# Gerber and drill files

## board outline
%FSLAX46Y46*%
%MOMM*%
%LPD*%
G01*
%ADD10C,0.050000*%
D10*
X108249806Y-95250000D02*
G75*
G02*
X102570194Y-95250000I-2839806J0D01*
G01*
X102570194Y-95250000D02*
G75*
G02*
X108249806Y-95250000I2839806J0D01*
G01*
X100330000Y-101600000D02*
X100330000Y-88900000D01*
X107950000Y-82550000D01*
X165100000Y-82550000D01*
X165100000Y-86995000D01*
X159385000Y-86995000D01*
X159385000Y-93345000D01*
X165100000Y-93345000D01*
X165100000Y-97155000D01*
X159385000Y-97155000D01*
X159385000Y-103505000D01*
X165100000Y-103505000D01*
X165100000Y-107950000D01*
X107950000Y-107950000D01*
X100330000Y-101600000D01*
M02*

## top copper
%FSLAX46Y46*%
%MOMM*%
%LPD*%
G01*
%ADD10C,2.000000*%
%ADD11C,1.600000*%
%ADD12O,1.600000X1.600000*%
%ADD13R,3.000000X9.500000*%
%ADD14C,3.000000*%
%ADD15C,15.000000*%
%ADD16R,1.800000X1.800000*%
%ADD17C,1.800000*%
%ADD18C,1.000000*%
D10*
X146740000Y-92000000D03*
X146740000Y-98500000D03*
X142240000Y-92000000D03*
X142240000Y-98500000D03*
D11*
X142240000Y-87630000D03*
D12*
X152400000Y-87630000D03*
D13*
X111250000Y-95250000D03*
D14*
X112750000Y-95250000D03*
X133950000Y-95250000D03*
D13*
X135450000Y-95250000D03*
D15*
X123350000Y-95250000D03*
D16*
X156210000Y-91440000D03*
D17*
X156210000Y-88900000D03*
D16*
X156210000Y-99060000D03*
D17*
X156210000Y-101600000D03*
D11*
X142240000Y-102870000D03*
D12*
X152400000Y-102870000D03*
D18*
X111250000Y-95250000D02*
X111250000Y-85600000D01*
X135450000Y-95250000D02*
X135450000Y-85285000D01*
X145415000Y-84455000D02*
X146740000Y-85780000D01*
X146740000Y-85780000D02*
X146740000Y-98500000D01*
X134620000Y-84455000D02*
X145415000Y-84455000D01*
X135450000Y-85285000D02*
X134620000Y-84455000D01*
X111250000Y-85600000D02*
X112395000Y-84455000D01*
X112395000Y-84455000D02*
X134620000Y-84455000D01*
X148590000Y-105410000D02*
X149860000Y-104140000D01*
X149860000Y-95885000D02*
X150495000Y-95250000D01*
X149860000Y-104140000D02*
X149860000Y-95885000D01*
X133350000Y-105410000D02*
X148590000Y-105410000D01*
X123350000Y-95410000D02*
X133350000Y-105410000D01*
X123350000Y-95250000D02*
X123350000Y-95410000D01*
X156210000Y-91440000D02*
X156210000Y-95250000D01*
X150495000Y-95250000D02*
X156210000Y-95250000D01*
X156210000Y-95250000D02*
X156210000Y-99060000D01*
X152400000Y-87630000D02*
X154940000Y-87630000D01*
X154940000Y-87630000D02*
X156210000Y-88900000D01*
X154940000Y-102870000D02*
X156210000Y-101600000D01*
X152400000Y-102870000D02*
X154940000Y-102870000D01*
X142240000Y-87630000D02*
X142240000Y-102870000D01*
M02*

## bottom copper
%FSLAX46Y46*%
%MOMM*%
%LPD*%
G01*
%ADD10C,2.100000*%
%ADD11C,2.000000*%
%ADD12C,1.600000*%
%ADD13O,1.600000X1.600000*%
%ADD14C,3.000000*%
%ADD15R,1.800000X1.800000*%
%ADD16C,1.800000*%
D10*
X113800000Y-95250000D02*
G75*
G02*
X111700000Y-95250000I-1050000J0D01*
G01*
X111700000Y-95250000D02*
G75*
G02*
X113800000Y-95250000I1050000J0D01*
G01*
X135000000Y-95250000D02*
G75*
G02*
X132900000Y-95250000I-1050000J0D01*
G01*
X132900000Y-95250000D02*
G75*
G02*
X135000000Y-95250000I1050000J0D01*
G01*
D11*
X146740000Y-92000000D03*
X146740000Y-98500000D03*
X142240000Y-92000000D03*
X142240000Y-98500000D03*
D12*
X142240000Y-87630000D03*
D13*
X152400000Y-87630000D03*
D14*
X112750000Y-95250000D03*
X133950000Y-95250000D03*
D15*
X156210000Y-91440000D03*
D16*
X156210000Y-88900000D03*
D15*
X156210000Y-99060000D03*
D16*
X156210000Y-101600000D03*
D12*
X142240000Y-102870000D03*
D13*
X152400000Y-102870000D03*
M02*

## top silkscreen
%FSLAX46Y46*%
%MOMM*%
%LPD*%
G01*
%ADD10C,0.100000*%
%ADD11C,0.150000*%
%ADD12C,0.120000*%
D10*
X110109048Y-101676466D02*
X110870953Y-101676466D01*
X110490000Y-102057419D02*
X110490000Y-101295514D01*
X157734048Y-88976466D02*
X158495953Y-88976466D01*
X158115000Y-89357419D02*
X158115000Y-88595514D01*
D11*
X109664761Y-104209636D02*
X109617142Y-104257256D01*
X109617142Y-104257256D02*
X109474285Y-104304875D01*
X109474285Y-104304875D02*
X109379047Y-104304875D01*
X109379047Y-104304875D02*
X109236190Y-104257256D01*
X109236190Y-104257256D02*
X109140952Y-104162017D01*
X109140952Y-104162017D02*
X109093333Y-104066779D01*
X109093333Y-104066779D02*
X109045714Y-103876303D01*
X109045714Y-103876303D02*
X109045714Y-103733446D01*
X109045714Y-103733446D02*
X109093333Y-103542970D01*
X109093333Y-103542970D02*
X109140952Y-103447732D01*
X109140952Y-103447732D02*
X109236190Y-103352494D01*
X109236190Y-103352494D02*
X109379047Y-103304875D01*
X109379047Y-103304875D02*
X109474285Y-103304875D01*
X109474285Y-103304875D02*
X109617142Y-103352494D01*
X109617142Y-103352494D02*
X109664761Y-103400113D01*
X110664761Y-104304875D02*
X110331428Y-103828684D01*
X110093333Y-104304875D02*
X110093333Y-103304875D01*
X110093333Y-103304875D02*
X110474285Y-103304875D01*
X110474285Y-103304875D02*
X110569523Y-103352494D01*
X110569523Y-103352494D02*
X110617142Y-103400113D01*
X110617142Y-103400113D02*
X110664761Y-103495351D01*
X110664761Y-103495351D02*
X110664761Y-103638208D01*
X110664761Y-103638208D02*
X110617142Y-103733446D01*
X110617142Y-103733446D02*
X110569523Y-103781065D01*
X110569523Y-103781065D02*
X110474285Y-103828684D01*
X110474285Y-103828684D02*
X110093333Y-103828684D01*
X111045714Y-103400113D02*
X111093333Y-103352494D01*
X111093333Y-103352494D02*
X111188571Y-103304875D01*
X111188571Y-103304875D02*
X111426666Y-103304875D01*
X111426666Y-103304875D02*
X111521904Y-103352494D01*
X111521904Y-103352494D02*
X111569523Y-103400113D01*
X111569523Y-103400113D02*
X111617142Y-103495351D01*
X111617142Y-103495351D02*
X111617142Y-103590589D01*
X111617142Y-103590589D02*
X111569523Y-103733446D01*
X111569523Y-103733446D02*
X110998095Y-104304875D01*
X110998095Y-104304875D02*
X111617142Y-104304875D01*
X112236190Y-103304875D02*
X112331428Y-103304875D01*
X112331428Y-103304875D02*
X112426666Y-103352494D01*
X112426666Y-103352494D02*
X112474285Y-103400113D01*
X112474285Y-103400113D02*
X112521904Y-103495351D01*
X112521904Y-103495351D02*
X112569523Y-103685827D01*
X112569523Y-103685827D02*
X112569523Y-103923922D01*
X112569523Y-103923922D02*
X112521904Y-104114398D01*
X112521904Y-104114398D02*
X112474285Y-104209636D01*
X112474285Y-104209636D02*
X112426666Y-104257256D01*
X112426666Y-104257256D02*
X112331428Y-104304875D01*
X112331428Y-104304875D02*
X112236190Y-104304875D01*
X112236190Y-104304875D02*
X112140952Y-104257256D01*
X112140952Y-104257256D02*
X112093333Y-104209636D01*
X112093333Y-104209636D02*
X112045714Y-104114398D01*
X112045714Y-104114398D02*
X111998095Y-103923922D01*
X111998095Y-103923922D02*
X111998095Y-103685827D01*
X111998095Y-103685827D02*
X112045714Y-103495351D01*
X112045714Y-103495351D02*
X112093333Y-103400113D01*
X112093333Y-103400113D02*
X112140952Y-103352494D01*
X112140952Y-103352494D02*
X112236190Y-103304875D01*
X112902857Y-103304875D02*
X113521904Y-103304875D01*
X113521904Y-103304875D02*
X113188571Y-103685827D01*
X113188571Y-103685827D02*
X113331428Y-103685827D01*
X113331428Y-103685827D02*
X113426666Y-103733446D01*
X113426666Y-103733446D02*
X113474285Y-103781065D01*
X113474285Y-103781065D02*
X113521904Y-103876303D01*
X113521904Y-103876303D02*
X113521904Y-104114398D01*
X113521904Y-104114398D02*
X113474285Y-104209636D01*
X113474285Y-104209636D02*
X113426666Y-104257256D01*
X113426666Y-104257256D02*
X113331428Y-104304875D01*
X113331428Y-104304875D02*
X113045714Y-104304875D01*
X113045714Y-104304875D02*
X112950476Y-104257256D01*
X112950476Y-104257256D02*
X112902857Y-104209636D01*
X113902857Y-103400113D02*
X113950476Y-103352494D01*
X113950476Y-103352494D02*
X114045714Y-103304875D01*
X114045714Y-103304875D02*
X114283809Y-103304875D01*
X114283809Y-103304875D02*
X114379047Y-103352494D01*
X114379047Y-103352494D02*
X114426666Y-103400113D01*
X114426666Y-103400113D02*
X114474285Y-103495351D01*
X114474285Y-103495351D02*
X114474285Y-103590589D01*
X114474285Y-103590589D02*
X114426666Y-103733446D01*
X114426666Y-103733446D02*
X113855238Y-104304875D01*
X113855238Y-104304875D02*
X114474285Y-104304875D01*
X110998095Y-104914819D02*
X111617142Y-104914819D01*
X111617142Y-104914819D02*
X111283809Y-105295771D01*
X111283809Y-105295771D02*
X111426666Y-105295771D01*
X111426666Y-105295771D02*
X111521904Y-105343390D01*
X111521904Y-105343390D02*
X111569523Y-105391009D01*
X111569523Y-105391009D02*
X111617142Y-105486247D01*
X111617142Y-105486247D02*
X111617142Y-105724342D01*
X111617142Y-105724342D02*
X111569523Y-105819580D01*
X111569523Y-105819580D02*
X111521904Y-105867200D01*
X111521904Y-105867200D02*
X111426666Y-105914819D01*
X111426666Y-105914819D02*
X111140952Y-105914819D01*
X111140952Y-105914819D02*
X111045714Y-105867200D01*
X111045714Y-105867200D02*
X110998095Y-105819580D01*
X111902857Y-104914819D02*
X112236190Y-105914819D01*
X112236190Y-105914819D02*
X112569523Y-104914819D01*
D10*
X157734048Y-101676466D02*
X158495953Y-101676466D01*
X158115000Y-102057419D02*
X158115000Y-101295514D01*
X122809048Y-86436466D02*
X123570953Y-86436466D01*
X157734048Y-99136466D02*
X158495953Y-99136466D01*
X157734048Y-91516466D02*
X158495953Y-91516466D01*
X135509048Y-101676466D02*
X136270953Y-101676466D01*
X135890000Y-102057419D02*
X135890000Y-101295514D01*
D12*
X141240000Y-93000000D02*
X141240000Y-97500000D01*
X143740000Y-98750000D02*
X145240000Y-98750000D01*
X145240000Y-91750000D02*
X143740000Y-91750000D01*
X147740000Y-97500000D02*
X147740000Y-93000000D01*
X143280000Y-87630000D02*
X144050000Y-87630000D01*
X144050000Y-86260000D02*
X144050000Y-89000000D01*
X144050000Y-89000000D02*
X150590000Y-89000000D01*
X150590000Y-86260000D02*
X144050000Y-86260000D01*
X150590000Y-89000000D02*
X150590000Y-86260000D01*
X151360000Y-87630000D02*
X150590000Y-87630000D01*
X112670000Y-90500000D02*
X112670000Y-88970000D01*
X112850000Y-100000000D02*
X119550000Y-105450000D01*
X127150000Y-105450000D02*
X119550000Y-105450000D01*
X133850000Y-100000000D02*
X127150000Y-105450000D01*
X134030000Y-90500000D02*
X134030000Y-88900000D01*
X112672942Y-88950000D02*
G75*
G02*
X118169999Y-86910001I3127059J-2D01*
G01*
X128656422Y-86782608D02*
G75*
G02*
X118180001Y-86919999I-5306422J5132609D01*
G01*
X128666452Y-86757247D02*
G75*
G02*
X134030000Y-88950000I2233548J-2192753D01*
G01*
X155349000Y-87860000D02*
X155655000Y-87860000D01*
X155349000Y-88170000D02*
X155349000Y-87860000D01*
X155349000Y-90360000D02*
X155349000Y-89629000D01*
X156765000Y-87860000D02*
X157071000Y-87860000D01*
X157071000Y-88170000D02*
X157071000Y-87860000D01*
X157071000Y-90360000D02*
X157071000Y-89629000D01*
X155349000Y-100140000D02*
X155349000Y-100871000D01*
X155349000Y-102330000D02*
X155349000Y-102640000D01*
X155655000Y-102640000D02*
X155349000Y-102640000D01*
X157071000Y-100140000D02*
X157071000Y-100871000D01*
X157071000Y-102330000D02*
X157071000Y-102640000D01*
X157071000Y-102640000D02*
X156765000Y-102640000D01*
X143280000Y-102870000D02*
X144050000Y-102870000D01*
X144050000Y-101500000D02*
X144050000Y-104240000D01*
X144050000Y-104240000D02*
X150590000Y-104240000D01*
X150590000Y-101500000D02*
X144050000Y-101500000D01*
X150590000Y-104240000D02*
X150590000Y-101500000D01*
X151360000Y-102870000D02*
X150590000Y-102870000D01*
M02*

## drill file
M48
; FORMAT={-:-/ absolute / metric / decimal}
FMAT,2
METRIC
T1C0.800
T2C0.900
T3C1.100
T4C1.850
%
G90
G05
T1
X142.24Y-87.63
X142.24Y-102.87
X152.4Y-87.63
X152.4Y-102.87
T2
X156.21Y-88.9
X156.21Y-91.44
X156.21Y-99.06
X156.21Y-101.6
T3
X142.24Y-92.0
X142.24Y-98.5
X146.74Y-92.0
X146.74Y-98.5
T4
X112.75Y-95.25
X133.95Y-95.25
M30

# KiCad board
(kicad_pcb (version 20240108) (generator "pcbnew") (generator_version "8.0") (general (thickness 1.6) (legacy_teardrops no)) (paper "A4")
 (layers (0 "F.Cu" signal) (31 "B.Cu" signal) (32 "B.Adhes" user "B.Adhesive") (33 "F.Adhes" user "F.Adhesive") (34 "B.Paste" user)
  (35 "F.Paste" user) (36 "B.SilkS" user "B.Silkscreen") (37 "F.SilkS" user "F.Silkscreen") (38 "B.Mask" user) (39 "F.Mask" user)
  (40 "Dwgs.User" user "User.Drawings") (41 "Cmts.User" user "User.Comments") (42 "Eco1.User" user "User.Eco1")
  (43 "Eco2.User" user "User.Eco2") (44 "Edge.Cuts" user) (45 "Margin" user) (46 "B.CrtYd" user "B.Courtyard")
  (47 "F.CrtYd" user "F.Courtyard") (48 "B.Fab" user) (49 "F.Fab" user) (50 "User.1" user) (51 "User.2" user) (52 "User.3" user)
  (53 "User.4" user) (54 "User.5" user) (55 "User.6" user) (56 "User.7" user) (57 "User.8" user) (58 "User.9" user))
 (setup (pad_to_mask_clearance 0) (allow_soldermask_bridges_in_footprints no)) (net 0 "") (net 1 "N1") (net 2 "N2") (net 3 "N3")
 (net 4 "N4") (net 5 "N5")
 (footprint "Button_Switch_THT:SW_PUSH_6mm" (layer "F.Cu") (at 146.74 92 -90)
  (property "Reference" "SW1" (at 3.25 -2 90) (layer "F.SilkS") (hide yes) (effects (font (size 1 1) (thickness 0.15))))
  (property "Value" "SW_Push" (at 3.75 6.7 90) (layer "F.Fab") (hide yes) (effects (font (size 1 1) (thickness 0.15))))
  (fp_line (start 1 5.5) (end 5.5 5.5) (stroke (width 0.12) (type solid)) (layer "F.SilkS"))
  (fp_line (start 6.75 3) (end 6.75 1.5) (stroke (width 0.12) (type solid)) (layer "F.SilkS"))
  (fp_line (start -0.25 1.5) (end -0.25 3) (stroke (width 0.12) (type solid)) (layer "F.SilkS"))
  (fp_line (start 5.5 -1) (end 1 -1) (stroke (width 0.12) (type solid)) (layer "F.SilkS"))
  (pad "1" thru_hole circle (at 0 0) (size 2 2) (drill 1.1) (layers "*.Cu" "*.Mask") (remove_unused_layers no) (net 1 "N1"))
  (pad "1" thru_hole circle (at 6.5 0) (size 2 2) (drill 1.1) (layers "*.Cu" "*.Mask") (remove_unused_layers no) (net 1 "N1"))
  (pad "2" thru_hole circle (at 0 4.5) (size 2 2) (drill 1.1) (layers "*.Cu" "*.Mask") (remove_unused_layers no) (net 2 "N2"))
  (pad "2" thru_hole circle (at 6.5 4.5) (size 2 2) (drill 1.1) (layers "*.Cu" "*.Mask") (remove_unused_layers no) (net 2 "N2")))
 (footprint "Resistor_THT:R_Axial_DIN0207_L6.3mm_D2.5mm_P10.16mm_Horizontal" (layer "F.Cu") (at 142.24 87.63)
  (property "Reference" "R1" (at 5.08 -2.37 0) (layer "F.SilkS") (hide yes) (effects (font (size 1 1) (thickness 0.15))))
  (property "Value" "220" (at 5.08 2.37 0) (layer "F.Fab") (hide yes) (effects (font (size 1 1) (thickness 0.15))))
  (fp_line (start 1.04 0) (end 1.81 0) (stroke (width 0.12) (type solid)) (layer "F.SilkS"))
  (fp_line (start 1.81 -1.37) (end 1.81 1.37) (stroke (width 0.12) (type solid)) (layer "F.SilkS"))
  (fp_line (start 1.81 1.37) (end 8.35 1.37) (stroke (width 0.12) (type solid)) (layer "F.SilkS"))
  (fp_line (start 8.35 -1.37) (end 1.81 -1.37) (stroke (width 0.12) (type solid)) (layer "F.SilkS"))
  (fp_line (start 8.35 1.37) (end 8.35 -1.37) (stroke (width 0.12) (type solid)) (layer "F.SilkS"))
  (fp_line (start 9.12 0) (end 8.35 0) (stroke (width 0.12) (type solid)) (layer "F.SilkS"))
  (pad "1" thru_hole circle (at 0 0) (size 1.6 1.6) (drill 0.8) (layers "*.Cu" "*.Mask") (remove_unused_layers no) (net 2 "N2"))
  (pad "2" thru_hole oval (at 10.16 0) (size 1.6 1.6) (drill 0.8) (layers "*.Cu" "*.Mask") (remove_unused_layers no) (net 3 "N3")))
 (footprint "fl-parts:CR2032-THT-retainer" (layer "F.Cu") (at 123.35 95.25)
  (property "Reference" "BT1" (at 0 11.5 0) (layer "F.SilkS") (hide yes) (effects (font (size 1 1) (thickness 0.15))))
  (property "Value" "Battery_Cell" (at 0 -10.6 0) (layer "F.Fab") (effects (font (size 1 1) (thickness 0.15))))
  (fp_circle (center -10.6 0) (end -8.6 0) (stroke (width 0.2) (type solid)) (fill solid) (layer "B.Cu"))
  (fp_circle (center 10.6 0) (end 12.6 0) (stroke (width 0.2) (type solid)) (fill solid) (layer "B.Cu"))
  (fp_line (start -10.68 -4.75) (end -10.68 -6.28) (stroke (width 0.12) (type solid)) (layer "F.SilkS"))
  (fp_line (start -10.5 4.75) (end -3.8 10.2) (stroke (width 0.12) (type solid)) (layer "F.SilkS"))
  (fp_line (start 3.8 10.2) (end -3.8 10.2) (stroke (width 0.12) (type solid)) (layer "F.SilkS"))
  (fp_line (start 10.5 4.75) (end 3.8 10.2) (stroke (width 0.12) (type solid)) (layer "F.SilkS"))
  (fp_line (start 10.68 -4.75) (end 10.68 -6.35) (stroke (width 0.12) (type solid)) (layer "F.SilkS"))
  (fp_arc (start -10.677058 -6.3) (mid -8.637972 -9.231689) (end -5.180001 -8.339999) (stroke (width 0.12) (type solid)) (layer "F.SilkS"))
  (fp_arc (start 5.306422 -8.467392) (mid 0.096808 -6.218103) (end -5.169999 -8.330001) (stroke (width 0.12) (type solid)) (layer "F.SilkS"))
  (fp_arc (start 5.316452 -8.492753) (mid 8.734461 -9.197232) (end 10.68 -6.3) (stroke (width 0.12) (type solid)) (layer "F.SilkS"))
  (pad "1" smd rect (at -12.1 0) (size 3 9.5) (layers "F.Cu" "F.Paste" "F.Mask") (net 1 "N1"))
  (pad "1" thru_hole circle (at -10.6 0) (size 3 3) (drill 1.85) (layers "*.Cu" "*.Mask") (remove_unused_layers no) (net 1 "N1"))
  (pad "1" thru_hole circle (at 10.6 0) (size 3 3) (drill 1.85) (layers "*.Cu" "*.Mask") (remove_unused_layers no) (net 1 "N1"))
  (pad "1" smd rect (at 12.1 0) (size 3 9.5) (layers "F.Cu" "F.Paste" "F.Mask") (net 1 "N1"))
  (pad "2" smd circle (at 0 0) (size 15 15) (layers "F.Cu" "F.Paste" "F.Mask") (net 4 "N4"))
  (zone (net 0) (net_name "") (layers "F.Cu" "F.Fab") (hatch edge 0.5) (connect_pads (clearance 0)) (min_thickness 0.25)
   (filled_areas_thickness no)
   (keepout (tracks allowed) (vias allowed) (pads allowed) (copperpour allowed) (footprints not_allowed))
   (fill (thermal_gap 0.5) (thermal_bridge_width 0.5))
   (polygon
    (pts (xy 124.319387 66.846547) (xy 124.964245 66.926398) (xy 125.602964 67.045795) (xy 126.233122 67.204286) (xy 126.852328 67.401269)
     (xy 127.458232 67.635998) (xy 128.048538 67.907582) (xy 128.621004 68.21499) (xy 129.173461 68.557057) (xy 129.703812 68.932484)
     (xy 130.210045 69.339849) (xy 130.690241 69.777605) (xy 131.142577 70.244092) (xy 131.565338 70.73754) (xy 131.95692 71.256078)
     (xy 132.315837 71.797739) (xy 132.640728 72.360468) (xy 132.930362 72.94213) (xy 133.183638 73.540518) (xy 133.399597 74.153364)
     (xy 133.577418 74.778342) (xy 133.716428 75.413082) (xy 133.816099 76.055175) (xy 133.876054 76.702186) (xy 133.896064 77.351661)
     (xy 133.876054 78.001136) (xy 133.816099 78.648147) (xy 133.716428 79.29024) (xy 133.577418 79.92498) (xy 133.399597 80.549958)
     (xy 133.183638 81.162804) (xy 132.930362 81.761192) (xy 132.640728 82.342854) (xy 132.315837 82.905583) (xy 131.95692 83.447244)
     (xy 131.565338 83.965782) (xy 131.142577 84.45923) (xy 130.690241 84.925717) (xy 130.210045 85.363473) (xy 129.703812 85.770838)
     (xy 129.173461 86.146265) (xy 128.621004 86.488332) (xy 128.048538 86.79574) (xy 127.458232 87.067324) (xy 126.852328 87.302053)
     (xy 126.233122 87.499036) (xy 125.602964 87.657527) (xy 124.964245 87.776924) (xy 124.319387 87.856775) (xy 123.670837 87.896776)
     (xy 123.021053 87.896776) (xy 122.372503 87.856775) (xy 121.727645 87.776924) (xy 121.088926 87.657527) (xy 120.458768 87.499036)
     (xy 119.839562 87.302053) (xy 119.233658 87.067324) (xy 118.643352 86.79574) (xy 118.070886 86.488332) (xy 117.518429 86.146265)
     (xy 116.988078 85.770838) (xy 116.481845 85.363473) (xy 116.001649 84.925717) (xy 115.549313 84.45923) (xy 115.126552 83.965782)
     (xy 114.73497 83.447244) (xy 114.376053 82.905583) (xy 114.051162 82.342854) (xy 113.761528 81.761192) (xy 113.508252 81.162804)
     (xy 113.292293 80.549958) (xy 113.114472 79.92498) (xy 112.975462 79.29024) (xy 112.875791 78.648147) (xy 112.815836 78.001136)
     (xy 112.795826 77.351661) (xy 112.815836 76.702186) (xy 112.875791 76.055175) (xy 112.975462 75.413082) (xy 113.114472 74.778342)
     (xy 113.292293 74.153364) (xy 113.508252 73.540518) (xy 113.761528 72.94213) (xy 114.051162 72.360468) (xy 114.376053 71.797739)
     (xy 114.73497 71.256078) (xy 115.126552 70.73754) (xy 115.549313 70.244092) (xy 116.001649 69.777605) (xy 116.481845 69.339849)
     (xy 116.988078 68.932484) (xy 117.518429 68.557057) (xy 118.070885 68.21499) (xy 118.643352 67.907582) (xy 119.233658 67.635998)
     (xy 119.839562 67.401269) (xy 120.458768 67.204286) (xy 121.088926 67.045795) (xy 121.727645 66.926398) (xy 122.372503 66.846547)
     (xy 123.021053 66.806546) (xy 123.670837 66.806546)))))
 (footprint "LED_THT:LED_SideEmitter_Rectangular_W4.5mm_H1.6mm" (layer "F.Cu") (at 156.21 91.44 90)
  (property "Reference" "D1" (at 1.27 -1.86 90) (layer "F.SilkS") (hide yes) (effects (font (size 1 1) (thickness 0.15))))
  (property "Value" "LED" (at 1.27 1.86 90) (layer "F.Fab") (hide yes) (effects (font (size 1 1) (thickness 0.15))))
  (fp_line (start 3.58 -0.861) (end 3.58 -0.555) (stroke (width 0.12) (type solid)) (layer "F.SilkS"))
  (fp_line (start 3.27 -0.861) (end 3.58 -0.861) (stroke (width 0.12) (type solid)) (layer "F.SilkS"))
  (fp_line (start 1.08 -0.861) (end 1.811 -0.861) (stroke (width 0.12) (type solid)) (layer "F.SilkS"))
  (fp_line (start 3.58 0.555) (end 3.58 0.861) (stroke (width 0.12) (type solid)) (layer "F.SilkS"))
  (fp_line (start 3.27 0.861) (end 3.58 0.861) (stroke (width 0.12) (type solid)) (layer "F.SilkS"))
  (fp_line (start 1.08 0.861) (end 1.811 0.861) (stroke (width 0.12) (type solid)) (layer "F.SilkS"))
  (pad "1" thru_hole rect (at 0 0 90) (size 1.8 1.8) (drill 0.9) (layers "*.Cu" "*.Mask") (remove_unused_layers no) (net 4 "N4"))
  (pad "2" thru_hole circle (at 2.54 0 90) (size 1.8 1.8) (drill 0.9) (layers "*.Cu" "*.Mask") (remove_unused_layers no) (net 3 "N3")))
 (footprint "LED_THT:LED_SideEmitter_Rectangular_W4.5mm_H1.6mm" (layer "F.Cu") (at 156.21 99.06 -90)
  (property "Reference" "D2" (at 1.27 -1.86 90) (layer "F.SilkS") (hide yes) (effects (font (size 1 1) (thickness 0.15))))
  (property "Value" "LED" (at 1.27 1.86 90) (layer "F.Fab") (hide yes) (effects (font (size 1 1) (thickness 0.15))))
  (fp_line (start 1.08 0.861) (end 1.811 0.861) (stroke (width 0.12) (type solid)) (layer "F.SilkS"))
  (fp_line (start 3.27 0.861) (end 3.58 0.861) (stroke (width 0.12) (type solid)) (layer "F.SilkS"))
  (fp_line (start 3.58 0.555) (end 3.58 0.861) (stroke (width 0.12) (type solid)) (layer "F.SilkS"))
  (fp_line (start 1.08 -0.861) (end 1.811 -0.861) (stroke (width 0.12) (type solid)) (layer "F.SilkS"))
  (fp_line (start 3.27 -0.861) (end 3.58 -0.861) (stroke (width 0.12) (type solid)) (layer "F.SilkS"))
  (fp_line (start 3.58 -0.861) (end 3.58 -0.555) (stroke (width 0.12) (type solid)) (layer "F.SilkS"))
  (pad "1" thru_hole rect (at 0 0 270) (size 1.8 1.8) (drill 0.9) (layers "*.Cu" "*.Mask") (remove_unused_layers no) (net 4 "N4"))
  (pad "2" thru_hole circle (at 2.54 0 270) (size 1.8 1.8) (drill 0.9) (layers "*.Cu" "*.Mask") (remove_unused_layers no) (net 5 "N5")))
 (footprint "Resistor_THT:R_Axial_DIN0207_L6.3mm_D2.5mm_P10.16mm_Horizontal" (layer "F.Cu") (at 142.24 102.87)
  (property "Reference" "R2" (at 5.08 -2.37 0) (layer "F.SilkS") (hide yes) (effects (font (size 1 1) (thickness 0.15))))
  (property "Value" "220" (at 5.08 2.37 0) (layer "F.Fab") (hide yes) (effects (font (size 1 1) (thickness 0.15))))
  (fp_line (start 1.04 0) (end 1.81 0) (stroke (width 0.12) (type solid)) (layer "F.SilkS"))
  (fp_line (start 1.81 -1.37) (end 1.81 1.37) (stroke (width 0.12) (type solid)) (layer "F.SilkS"))
  (fp_line (start 1.81 1.37) (end 8.35 1.37) (stroke (width 0.12) (type solid)) (layer "F.SilkS"))
  (fp_line (start 8.35 -1.37) (end 1.81 -1.37) (stroke (width 0.12) (type solid)) (layer "F.SilkS"))
  (fp_line (start 8.35 1.37) (end 8.35 -1.37) (stroke (width 0.12) (type solid)) (layer "F.SilkS"))
  (fp_line (start 9.12 0) (end 8.35 0) (stroke (width 0.12) (type solid)) (layer "F.SilkS"))
  (pad "1" thru_hole circle (at 0 0) (size 1.6 1.6) (drill 0.8) (layers "*.Cu" "*.Mask") (remove_unused_layers no) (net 2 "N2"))
  (pad "2" thru_hole oval (at 10.16 0) (size 1.6 1.6) (drill 0.8) (layers "*.Cu" "*.Mask") (remove_unused_layers no) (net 5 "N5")))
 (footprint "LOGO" (layer "B.Cu") (at 124.46 100.33 180)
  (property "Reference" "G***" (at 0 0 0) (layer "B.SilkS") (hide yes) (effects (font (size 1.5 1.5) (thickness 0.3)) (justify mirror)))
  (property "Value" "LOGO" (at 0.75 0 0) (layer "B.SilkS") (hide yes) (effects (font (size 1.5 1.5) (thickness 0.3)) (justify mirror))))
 (gr_circle (center 105.41 95.25) (end 102.87 93.98) (stroke (width 0.05) (type default)) (fill none) (layer "Edge.Cuts"))
 (gr_poly
  (pts (xy 100.33 101.6) (xy 100.33 88.9) (xy 107.95 82.55) (xy 165.1 82.55) (xy 165.1 86.995) (xy 159.385 86.995) (xy 159.385 93.345)
   (xy 165.1 93.345) (xy 165.1 97.155) (xy 159.385 97.155) (xy 159.385 103.505) (xy 165.1 103.505) (xy 165.1 107.95) (xy 107.95 107.95))
  (stroke (width 0.05) (type solid)) (fill none) (layer "Edge.Cuts"))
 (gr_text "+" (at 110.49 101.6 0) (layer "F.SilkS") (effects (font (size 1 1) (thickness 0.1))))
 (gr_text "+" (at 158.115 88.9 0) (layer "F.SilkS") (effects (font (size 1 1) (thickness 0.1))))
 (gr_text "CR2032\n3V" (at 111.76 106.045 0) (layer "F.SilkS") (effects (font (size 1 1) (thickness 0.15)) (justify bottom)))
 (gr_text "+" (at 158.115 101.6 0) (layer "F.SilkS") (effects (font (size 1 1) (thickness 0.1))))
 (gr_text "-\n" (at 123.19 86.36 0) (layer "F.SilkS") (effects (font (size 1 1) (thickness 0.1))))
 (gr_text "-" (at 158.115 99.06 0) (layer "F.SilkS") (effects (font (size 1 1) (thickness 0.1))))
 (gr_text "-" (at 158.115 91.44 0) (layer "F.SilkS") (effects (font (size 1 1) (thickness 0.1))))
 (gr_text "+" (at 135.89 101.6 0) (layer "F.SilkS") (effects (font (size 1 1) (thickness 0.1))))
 (segment (start 111.25 95.25) (end 111.25 85.6) (width 1) (layer "F.Cu") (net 1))
 (segment (start 135.45 95.25) (end 135.45 85.285) (width 1) (layer "F.Cu") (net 1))
 (segment (start 145.415 84.455) (end 146.74 85.78) (width 1) (layer "F.Cu") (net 1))
 (segment (start 146.74 85.78) (end 146.74 98.5) (width 1) (layer "F.Cu") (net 1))
 (segment (start 134.62 84.455) (end 145.415 84.455) (width 1) (layer "F.Cu") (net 1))
 (segment (start 135.45 85.285) (end 134.62 84.455) (width 1) (layer "F.Cu") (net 1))
 (segment (start 111.25 85.6) (end 112.395 84.455) (width 1) (layer "F.Cu") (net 1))
 (segment (start 112.395 84.455) (end 134.62 84.455) (width 1) (layer "F.Cu") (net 1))
 (segment (start 148.59 105.41) (end 149.86 104.14) (width 1) (layer "F.Cu") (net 4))
 (segment (start 149.86 95.885) (end 150.495 95.25) (width 1) (layer "F.Cu") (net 4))
 (segment (start 149.86 104.14) (end 149.86 95.885) (width 1) (layer "F.Cu") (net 4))
 (segment (start 133.35 105.41) (end 148.59 105.41) (width 1) (layer "F.Cu") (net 4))
 (segment (start 123.35 95.41) (end 133.35 105.41) (width 1) (layer "F.Cu") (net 4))
 (segment (start 123.35 95.25) (end 123.35 95.41) (width 1) (layer "F.Cu") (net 4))
 (segment (start 156.21 91.44) (end 156.21 95.25) (width 1) (layer "F.Cu") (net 4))
 (segment (start 150.495 95.25) (end 156.21 95.25) (width 1) (layer "F.Cu") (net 4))
 (segment (start 156.21 95.25) (end 156.21 99.06) (width 1) (layer "F.Cu") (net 4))
 (segment (start 152.4 87.63) (end 154.94 87.63) (width 1) (layer "F.Cu") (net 3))
 (segment (start 154.94 87.63) (end 156.21 88.9) (width 1) (layer "F.Cu") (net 3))
 (segment (start 154.94 102.87) (end 156.21 101.6) (width 1) (layer "F.Cu") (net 5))
 (segment (start 152.4 102.87) (end 154.94 102.87) (width 1) (layer "F.Cu") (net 5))
 (segment (start 142.24 87.63) (end 142.24 102.87) (width 1) (layer "F.Cu") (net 2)))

